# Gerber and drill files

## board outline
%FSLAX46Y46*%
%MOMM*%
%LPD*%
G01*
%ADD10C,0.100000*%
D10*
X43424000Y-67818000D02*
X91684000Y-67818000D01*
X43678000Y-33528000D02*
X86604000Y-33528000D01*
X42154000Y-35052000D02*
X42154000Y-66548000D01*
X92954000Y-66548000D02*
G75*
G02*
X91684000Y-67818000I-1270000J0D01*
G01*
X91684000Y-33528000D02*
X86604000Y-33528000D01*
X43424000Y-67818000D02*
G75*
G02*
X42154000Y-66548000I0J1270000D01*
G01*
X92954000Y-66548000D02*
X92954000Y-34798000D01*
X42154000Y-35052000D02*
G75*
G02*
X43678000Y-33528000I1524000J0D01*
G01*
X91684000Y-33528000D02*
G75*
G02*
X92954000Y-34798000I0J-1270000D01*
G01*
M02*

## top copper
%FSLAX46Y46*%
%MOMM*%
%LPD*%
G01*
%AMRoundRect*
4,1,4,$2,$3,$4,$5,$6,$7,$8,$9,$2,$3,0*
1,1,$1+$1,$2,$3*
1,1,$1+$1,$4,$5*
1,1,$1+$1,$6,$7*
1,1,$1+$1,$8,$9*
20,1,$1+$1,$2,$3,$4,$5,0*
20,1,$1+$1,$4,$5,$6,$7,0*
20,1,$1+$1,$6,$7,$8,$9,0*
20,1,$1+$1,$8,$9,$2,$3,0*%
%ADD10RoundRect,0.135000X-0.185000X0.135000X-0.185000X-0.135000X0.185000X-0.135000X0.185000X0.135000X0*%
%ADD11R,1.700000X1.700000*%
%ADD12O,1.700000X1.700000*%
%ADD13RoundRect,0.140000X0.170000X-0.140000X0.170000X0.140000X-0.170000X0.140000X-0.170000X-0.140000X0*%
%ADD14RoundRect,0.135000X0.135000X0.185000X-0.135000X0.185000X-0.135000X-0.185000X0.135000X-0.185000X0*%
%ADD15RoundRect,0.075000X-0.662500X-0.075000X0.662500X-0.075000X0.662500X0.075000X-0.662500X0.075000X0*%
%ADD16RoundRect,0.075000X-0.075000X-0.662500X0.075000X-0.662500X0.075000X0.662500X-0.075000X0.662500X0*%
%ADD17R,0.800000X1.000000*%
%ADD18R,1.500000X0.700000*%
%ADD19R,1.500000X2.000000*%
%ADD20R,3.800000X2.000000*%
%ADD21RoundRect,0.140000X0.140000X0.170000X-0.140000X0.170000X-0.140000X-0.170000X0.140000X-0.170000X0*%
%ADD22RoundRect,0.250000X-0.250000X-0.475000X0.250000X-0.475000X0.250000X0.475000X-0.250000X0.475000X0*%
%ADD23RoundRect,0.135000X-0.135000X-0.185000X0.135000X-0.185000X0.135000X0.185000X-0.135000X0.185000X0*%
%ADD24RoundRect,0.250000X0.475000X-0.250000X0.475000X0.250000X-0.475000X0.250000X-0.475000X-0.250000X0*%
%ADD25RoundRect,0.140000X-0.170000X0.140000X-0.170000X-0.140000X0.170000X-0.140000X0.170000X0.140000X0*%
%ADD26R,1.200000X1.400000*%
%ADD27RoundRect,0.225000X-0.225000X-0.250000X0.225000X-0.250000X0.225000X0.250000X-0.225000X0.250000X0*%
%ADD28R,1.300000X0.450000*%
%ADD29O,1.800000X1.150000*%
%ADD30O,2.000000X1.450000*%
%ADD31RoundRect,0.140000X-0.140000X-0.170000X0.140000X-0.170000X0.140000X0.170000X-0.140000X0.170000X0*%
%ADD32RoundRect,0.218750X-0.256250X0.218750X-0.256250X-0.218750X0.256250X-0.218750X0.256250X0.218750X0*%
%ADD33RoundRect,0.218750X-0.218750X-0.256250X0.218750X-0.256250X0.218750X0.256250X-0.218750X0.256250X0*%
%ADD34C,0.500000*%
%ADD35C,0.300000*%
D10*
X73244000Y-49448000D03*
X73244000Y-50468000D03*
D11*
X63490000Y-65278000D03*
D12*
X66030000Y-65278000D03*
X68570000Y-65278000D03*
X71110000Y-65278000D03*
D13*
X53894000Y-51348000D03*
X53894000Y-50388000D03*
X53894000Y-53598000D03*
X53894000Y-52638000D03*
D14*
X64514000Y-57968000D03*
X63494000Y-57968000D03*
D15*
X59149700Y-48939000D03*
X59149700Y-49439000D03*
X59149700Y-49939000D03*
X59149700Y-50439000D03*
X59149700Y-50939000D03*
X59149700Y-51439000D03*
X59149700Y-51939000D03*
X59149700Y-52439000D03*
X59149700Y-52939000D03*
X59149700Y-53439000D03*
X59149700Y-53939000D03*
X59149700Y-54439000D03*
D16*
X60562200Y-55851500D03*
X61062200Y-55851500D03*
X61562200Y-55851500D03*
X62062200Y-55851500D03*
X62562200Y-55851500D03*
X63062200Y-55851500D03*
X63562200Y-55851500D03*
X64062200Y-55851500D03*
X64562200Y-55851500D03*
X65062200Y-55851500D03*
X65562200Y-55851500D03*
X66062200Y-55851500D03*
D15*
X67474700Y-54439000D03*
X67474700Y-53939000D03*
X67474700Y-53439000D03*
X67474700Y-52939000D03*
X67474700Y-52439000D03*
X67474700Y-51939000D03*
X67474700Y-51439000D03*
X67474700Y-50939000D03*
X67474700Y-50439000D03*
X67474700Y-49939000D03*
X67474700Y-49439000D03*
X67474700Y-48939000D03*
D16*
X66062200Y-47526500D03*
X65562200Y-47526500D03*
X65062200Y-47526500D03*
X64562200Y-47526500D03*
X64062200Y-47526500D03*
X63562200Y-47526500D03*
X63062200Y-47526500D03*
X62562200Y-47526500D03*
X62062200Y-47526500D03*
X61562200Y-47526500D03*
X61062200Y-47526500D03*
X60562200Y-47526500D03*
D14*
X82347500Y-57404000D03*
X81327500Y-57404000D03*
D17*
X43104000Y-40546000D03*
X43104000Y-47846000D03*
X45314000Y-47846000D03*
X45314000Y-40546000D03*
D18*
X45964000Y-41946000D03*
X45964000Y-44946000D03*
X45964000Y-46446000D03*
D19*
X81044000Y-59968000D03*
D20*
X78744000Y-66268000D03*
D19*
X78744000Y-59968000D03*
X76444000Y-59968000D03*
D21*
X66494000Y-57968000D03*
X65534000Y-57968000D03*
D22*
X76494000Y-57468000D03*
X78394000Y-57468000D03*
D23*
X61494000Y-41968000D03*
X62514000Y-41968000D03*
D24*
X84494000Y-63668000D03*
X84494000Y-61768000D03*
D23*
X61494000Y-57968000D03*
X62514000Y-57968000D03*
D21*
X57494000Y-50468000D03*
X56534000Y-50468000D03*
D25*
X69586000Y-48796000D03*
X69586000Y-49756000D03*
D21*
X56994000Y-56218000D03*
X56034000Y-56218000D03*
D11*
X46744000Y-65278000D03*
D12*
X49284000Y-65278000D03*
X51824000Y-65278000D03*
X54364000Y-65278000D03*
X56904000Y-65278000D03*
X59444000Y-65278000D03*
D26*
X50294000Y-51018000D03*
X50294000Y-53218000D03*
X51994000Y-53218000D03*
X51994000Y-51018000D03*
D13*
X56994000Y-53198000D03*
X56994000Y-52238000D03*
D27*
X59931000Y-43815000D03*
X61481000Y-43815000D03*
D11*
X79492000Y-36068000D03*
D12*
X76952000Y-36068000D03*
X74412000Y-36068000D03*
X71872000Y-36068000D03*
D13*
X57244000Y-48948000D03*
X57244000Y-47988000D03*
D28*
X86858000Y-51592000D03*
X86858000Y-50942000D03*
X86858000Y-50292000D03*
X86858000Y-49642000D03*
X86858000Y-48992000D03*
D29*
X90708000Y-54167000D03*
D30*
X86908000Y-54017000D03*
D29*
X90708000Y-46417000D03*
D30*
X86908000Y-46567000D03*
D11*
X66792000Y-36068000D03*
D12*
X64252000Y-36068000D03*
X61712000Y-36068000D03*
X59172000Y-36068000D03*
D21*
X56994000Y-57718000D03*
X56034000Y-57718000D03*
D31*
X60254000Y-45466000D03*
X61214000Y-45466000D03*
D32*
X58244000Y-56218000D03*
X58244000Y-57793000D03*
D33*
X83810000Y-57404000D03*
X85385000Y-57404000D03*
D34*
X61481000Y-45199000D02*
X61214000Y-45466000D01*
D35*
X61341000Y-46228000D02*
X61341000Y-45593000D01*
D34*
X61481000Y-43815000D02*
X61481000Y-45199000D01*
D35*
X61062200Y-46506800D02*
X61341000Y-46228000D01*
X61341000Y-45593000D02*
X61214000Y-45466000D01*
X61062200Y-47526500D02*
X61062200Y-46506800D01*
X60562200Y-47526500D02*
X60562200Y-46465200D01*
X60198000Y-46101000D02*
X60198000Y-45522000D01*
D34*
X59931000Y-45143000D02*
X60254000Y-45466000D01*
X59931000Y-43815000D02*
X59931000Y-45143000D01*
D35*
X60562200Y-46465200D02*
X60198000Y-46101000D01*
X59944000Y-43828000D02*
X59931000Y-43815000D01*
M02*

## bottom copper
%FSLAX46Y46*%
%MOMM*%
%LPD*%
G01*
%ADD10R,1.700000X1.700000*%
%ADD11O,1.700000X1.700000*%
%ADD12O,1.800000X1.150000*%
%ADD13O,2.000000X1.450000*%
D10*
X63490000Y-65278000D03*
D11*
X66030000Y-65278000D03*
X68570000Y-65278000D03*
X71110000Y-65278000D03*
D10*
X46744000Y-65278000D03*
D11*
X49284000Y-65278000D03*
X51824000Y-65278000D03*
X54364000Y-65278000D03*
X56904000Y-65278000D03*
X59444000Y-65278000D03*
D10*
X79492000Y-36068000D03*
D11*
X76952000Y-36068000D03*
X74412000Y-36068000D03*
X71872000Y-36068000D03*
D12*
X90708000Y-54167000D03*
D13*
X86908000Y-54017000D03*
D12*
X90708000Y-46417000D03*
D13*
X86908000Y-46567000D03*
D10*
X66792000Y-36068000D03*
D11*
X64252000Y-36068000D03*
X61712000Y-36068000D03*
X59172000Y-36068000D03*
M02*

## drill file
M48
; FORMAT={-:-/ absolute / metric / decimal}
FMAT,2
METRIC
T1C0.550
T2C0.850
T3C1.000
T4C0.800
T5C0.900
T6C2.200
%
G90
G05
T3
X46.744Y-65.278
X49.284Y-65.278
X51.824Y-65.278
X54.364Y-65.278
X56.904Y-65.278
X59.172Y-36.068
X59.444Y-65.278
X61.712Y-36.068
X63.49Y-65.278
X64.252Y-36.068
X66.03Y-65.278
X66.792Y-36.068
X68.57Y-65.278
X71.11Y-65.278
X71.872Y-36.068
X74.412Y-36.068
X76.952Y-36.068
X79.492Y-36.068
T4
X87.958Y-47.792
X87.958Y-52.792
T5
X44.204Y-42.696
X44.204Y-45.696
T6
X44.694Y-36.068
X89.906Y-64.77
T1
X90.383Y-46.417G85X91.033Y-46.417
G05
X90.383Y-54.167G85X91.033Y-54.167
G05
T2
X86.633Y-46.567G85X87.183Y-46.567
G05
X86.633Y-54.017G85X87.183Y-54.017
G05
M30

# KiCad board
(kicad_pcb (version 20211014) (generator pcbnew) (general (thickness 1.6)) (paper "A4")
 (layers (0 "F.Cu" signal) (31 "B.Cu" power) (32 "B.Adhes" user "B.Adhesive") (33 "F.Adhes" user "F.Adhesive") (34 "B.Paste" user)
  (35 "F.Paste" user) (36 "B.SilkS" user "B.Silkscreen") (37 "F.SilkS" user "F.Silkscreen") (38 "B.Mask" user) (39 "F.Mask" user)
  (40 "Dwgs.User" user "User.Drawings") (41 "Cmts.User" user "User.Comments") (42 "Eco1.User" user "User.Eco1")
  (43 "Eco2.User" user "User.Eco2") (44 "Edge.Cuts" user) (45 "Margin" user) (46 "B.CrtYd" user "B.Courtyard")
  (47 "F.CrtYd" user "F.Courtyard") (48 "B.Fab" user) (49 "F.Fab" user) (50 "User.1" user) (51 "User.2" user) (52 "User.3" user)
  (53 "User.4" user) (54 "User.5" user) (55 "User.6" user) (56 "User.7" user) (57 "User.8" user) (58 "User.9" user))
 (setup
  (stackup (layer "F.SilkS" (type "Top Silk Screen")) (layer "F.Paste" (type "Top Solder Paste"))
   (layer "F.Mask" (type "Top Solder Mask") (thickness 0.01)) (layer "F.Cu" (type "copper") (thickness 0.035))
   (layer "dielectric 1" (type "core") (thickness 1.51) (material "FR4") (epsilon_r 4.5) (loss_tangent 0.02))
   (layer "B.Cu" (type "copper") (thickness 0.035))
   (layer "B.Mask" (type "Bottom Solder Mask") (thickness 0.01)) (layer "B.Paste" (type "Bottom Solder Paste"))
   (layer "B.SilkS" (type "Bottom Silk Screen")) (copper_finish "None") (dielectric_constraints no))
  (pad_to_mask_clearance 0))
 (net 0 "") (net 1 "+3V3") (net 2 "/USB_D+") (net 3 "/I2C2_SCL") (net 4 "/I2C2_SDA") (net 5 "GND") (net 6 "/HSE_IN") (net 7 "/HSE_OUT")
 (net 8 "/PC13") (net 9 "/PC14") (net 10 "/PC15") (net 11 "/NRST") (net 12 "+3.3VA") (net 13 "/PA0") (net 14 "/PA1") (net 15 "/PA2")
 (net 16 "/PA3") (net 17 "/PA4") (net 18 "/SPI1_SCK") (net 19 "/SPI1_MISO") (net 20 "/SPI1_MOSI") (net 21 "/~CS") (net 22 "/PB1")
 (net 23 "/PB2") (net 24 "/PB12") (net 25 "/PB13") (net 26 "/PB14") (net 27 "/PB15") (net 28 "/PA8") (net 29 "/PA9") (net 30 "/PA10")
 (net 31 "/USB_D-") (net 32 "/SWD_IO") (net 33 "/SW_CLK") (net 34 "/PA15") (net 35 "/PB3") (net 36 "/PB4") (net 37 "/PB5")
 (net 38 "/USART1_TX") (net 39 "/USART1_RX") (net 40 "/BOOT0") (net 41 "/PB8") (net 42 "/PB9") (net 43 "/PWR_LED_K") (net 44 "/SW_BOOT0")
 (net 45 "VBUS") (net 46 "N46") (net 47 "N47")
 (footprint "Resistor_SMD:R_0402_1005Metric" (layer "F.Cu") (at 73.244 49.958 -90)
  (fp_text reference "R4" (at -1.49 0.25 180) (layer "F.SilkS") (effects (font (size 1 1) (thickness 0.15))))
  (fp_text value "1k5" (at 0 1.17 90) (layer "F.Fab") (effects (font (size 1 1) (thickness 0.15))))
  (pad "1" smd roundrect locked (at -0.51 0 270) (size 0.54 0.64) (layers "F.Cu" "F.Paste" "F.Mask") (roundrect_rratio 0.25) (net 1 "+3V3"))
  (pad "2" smd roundrect locked (at 0.51 0 270) (size 0.54 0.64) (layers "F.Cu" "F.Paste" "F.Mask") (roundrect_rratio 0.25)
   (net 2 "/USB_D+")))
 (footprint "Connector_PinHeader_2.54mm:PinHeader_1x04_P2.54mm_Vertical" (layer "F.Cu") (at 63.49 65.278 90)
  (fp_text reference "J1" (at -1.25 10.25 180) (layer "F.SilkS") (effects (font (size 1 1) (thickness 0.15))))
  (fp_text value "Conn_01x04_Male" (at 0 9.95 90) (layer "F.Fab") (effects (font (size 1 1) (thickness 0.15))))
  (pad "1" thru_hole rect locked (at 0 0 90) (size 1.7 1.7) (drill 1) (layers *.Cu *.Mask) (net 1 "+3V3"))
  (pad "2" thru_hole oval locked (at 0 2.54 90) (size 1.7 1.7) (drill 1) (layers *.Cu *.Mask) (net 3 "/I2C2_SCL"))
  (pad "3" thru_hole oval locked (at 0 5.08 90) (size 1.7 1.7) (drill 1) (layers *.Cu *.Mask) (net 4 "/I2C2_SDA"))
  (pad "4" thru_hole oval locked (at 0 7.62 90) (size 1.7 1.7) (drill 1) (layers *.Cu *.Mask) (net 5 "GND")))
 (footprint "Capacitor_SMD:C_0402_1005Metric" (layer "F.Cu") (at 53.894 50.868 90)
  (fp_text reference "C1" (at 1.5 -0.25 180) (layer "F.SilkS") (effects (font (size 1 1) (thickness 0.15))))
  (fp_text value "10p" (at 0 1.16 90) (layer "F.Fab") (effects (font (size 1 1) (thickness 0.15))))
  (pad "1" smd roundrect locked (at -0.48 0 90) (size 0.56 0.62) (layers "F.Cu" "F.Paste" "F.Mask") (roundrect_rratio 0.25)
   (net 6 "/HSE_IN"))
  (pad "2" smd roundrect locked (at 0.48 0 90) (size 0.56 0.62) (layers "F.Cu" "F.Paste" "F.Mask") (roundrect_rratio 0.25) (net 5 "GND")))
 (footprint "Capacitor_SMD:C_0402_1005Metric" (layer "F.Cu") (at 53.894 53.118 90)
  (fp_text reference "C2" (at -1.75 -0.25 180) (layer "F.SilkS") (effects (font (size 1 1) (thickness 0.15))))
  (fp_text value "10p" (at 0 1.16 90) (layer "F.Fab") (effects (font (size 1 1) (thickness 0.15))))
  (pad "1" smd roundrect locked (at -0.48 0 90) (size 0.56 0.62) (layers "F.Cu" "F.Paste" "F.Mask") (roundrect_rratio 0.25)
   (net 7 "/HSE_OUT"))
  (pad "2" smd roundrect locked (at 0.48 0 90) (size 0.56 0.62) (layers "F.Cu" "F.Paste" "F.Mask") (roundrect_rratio 0.25) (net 5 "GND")))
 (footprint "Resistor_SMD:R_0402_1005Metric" (layer "F.Cu") (at 64.004 57.968 180)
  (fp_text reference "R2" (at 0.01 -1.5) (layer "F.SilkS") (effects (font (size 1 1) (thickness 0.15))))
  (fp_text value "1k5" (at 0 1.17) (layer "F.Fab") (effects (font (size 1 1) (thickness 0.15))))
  (pad "1" smd roundrect locked (at -0.51 0 180) (size 0.54 0.64) (layers "F.Cu" "F.Paste" "F.Mask") (roundrect_rratio 0.25) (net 1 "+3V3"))
  (pad "2" smd roundrect locked (at 0.51 0 180) (size 0.54 0.64) (layers "F.Cu" "F.Paste" "F.Mask") (roundrect_rratio 0.25)
   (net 4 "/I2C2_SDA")))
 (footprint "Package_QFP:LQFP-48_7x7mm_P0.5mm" (layer "F.Cu") (at 63.3122 51.689)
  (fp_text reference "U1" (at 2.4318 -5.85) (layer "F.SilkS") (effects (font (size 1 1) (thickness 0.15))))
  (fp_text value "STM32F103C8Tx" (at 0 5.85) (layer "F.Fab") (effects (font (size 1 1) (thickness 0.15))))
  (pad "1" smd roundrect locked (at -4.1625 -2.75) (size 1.475 0.3) (layers "F.Cu" "F.Paste" "F.Mask") (roundrect_rratio 0.25)
   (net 1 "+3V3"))
  (pad "2" smd roundrect locked (at -4.1625 -2.25) (size 1.475 0.3) (layers "F.Cu" "F.Paste" "F.Mask") (roundrect_rratio 0.25)
   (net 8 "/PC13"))
  (pad "3" smd roundrect locked (at -4.1625 -1.75) (size 1.475 0.3) (layers "F.Cu" "F.Paste" "F.Mask") (roundrect_rratio 0.25)
   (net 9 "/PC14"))
  (pad "4" smd roundrect locked (at -4.1625 -1.25) (size 1.475 0.3) (layers "F.Cu" "F.Paste" "F.Mask") (roundrect_rratio 0.25)
   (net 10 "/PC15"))
  (pad "5" smd roundrect locked (at -4.1625 -0.75) (size 1.475 0.3) (layers "F.Cu" "F.Paste" "F.Mask") (roundrect_rratio 0.25)
   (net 6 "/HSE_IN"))
  (pad "6" smd roundrect locked (at -4.1625 -0.25) (size 1.475 0.3) (layers "F.Cu" "F.Paste" "F.Mask") (roundrect_rratio 0.25)
   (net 7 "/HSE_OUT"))
  (pad "7" smd roundrect locked (at -4.1625 0.25) (size 1.475 0.3) (layers "F.Cu" "F.Paste" "F.Mask") (roundrect_rratio 0.25)
   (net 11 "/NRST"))
  (pad "8" smd roundrect locked (at -4.1625 0.75) (size 1.475 0.3) (layers "F.Cu" "F.Paste" "F.Mask") (roundrect_rratio 0.25) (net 5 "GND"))
  (pad "9" smd roundrect locked (at -4.1625 1.25) (size 1.475 0.3) (layers "F.Cu" "F.Paste" "F.Mask") (roundrect_rratio 0.25)
   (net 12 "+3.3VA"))
  (pad "10" smd roundrect locked (at -4.1625 1.75) (size 1.475 0.3) (layers "F.Cu" "F.Paste" "F.Mask") (roundrect_rratio 0.25)
   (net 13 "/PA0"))
  (pad "11" smd roundrect locked (at -4.1625 2.25) (size 1.475 0.3) (layers "F.Cu" "F.Paste" "F.Mask") (roundrect_rratio 0.25)
   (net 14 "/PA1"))
  (pad "12" smd roundrect locked (at -4.1625 2.75) (size 1.475 0.3) (layers "F.Cu" "F.Paste" "F.Mask") (roundrect_rratio 0.25)
   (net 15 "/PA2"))
  (pad "13" smd roundrect locked (at -2.75 4.1625) (size 0.3 1.475) (layers "F.Cu" "F.Paste" "F.Mask") (roundrect_rratio 0.25)
   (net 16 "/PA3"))
  (pad "14" smd roundrect locked (at -2.25 4.1625) (size 0.3 1.475) (layers "F.Cu" "F.Paste" "F.Mask") (roundrect_rratio 0.25)
   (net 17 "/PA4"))
  (pad "15" smd roundrect locked (at -1.75 4.1625) (size 0.3 1.475) (layers "F.Cu" "F.Paste" "F.Mask") (roundrect_rratio 0.25)
   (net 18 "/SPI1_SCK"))
  (pad "16" smd roundrect locked (at -1.25 4.1625) (size 0.3 1.475) (layers "F.Cu" "F.Paste" "F.Mask") (roundrect_rratio 0.25)
   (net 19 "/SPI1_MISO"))
  (pad "17" smd roundrect locked (at -0.75 4.1625) (size 0.3 1.475) (layers "F.Cu" "F.Paste" "F.Mask") (roundrect_rratio 0.25)
   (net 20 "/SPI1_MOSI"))
  (pad "18" smd roundrect locked (at -0.25 4.1625) (size 0.3 1.475) (layers "F.Cu" "F.Paste" "F.Mask") (roundrect_rratio 0.25)
   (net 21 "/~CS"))
  (pad "19" smd roundrect locked (at 0.25 4.1625) (size 0.3 1.475) (layers "F.Cu" "F.Paste" "F.Mask") (roundrect_rratio 0.25)
   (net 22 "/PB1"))
  (pad "20" smd roundrect locked (at 0.75 4.1625) (size 0.3 1.475) (layers "F.Cu" "F.Paste" "F.Mask") (roundrect_rratio 0.25)
   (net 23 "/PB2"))
  (pad "21" smd roundrect locked (at 1.25 4.1625) (size 0.3 1.475) (layers "F.Cu" "F.Paste" "F.Mask") (roundrect_rratio 0.25)
   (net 3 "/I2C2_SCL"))
  (pad "22" smd roundrect locked (at 1.75 4.1625) (size 0.3 1.475) (layers "F.Cu" "F.Paste" "F.Mask") (roundrect_rratio 0.25)
   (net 4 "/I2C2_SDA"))
  (pad "23" smd roundrect locked (at 2.25 4.1625) (size 0.3 1.475) (layers "F.Cu" "F.Paste" "F.Mask") (roundrect_rratio 0.25) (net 5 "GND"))
  (pad "24" smd roundrect locked (at 2.75 4.1625) (size 0.3 1.475) (layers "F.Cu" "F.Paste" "F.Mask") (roundrect_rratio 0.25) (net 1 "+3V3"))
  (pad "25" smd roundrect locked (at 4.1625 2.75) (size 1.475 0.3) (layers "F.Cu" "F.Paste" "F.Mask") (roundrect_rratio 0.25)
   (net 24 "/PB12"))
  (pad "26" smd roundrect locked (at 4.1625 2.25) (size 1.475 0.3) (layers "F.Cu" "F.Paste" "F.Mask") (roundrect_rratio 0.25)
   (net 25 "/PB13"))
  (pad "27" smd roundrect locked (at 4.1625 1.75) (size 1.475 0.3) (layers "F.Cu" "F.Paste" "F.Mask") (roundrect_rratio 0.25)
   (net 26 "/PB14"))
  (pad "28" smd roundrect locked (at 4.1625 1.25) (size 1.475 0.3) (layers "F.Cu" "F.Paste" "F.Mask") (roundrect_rratio 0.25)
   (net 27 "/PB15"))
  (pad "29" smd roundrect locked (at 4.1625 0.75) (size 1.475 0.3) (layers "F.Cu" "F.Paste" "F.Mask") (roundrect_rratio 0.25)
   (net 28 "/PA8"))
  (pad "30" smd roundrect locked (at 4.1625 0.25) (size 1.475 0.3) (layers "F.Cu" "F.Paste" "F.Mask") (roundrect_rratio 0.25)
   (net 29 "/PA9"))
  (pad "31" smd roundrect locked (at 4.1625 -0.25) (size 1.475 0.3) (layers "F.Cu" "F.Paste" "F.Mask") (roundrect_rratio 0.25)
   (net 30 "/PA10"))
  (pad "32" smd roundrect locked (at 4.1625 -0.75) (size 1.475 0.3) (layers "F.Cu" "F.Paste" "F.Mask") (roundrect_rratio 0.25)
   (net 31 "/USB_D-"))
  (pad "33" smd roundrect locked (at 4.1625 -1.25) (size 1.475 0.3) (layers "F.Cu" "F.Paste" "F.Mask") (roundrect_rratio 0.25)
   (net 2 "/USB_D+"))
  (pad "34" smd roundrect locked (at 4.1625 -1.75) (size 1.475 0.3) (layers "F.Cu" "F.Paste" "F.Mask") (roundrect_rratio 0.25)
   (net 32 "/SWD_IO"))
  (pad "35" smd roundrect locked (at 4.1625 -2.25) (size 1.475 0.3) (layers "F.Cu" "F.Paste" "F.Mask") (roundrect_rratio 0.25) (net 5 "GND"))
  (pad "36" smd roundrect locked (at 4.1625 -2.75) (size 1.475 0.3) (layers "F.Cu" "F.Paste" "F.Mask") (roundrect_rratio 0.25)
   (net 1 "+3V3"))
  (pad "37" smd roundrect locked (at 2.75 -4.1625) (size 0.3 1.475) (layers "F.Cu" "F.Paste" "F.Mask") (roundrect_rratio 0.25)
   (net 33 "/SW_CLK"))
  (pad "38" smd roundrect locked (at 2.25 -4.1625) (size 0.3 1.475) (layers "F.Cu" "F.Paste" "F.Mask") (roundrect_rratio 0.25)
   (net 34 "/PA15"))
  (pad "39" smd roundrect locked (at 1.75 -4.1625) (size 0.3 1.475) (layers "F.Cu" "F.Paste" "F.Mask") (roundrect_rratio 0.25)
   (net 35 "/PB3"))
  (pad "40" smd roundrect locked (at 1.25 -4.1625) (size 0.3 1.475) (layers "F.Cu" "F.Paste" "F.Mask") (roundrect_rratio 0.25)
   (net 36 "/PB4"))
  (pad "41" smd roundrect locked (at 0.75 -4.1625) (size 0.3 1.475) (layers "F.Cu" "F.Paste" "F.Mask") (roundrect_rratio 0.25)
   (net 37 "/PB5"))
  (pad "42" smd roundrect locked (at 0.25 -4.1625) (size 0.3 1.475) (layers "F.Cu" "F.Paste" "F.Mask") (roundrect_rratio 0.25)
   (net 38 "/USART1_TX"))
  (pad "43" smd roundrect locked (at -0.25 -4.1625) (size 0.3 1.475) (layers "F.Cu" "F.Paste" "F.Mask") (roundrect_rratio 0.25)
   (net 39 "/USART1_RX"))
  (pad "44" smd roundrect locked (at -0.75 -4.1625) (size 0.3 1.475) (layers "F.Cu" "F.Paste" "F.Mask") (roundrect_rratio 0.25)
   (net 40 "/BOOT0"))
  (pad "45" smd roundrect locked (at -1.25 -4.1625) (size 0.3 1.475) (layers "F.Cu" "F.Paste" "F.Mask") (roundrect_rratio 0.25)
   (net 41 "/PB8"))
  (pad "46" smd roundrect locked (at -1.75 -4.1625) (size 0.3 1.475) (layers "F.Cu" "F.Paste" "F.Mask") (roundrect_rratio 0.25)
   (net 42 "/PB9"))
  (pad "47" smd roundrect locked (at -2.25 -4.1625) (size 0.3 1.475) (layers "F.Cu" "F.Paste" "F.Mask") (roundrect_rratio 0.25)
   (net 5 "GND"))
  (pad "48" smd roundrect locked (at -2.75 -4.1625) (size 0.3 1.475) (layers "F.Cu" "F.Paste" "F.Mask") (roundrect_rratio 0.25)
   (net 1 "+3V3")))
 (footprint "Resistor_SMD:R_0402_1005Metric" (layer "F.Cu") (at 81.8375 57.404 180)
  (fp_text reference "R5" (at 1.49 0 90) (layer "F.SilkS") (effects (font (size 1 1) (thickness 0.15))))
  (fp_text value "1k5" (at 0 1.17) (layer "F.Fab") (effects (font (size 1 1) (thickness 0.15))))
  (pad "1" smd roundrect locked (at -0.51 0 180) (size 0.54 0.64) (layers "F.Cu" "F.Paste" "F.Mask") (roundrect_rratio 0.25)
   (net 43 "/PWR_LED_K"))
  (pad "2" smd roundrect locked (at 0.51 0 180) (size 0.54 0.64) (layers "F.Cu" "F.Paste" "F.Mask") (roundrect_rratio 0.25) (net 5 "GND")))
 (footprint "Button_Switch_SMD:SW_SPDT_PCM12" (layer "F.Cu") (at 44.534 44.196 -90)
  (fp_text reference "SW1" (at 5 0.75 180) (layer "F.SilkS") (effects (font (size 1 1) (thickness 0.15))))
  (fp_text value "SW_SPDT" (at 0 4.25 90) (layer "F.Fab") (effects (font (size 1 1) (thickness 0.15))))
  (pad "" smd rect (at -3.65 1.43 270) (size 1 0.8) (layers "F.Cu" "F.Paste" "F.Mask"))
  (pad "" smd rect (at 3.65 1.43 270) (size 1 0.8) (layers "F.Cu" "F.Paste" "F.Mask"))
  (pad "" np_thru_hole circle (at 1.5 0.33 270) (size 0.9 0.9) (drill 0.9) (layers *.Cu *.Mask))
  (pad "" smd rect (at 3.65 -0.78 270) (size 1 0.8) (layers "F.Cu" "F.Paste" "F.Mask"))
  (pad "" smd rect (at -3.65 -0.78 270) (size 1 0.8) (layers "F.Cu" "F.Paste" "F.Mask"))
  (pad "" np_thru_hole circle (at -1.5 0.33 270) (size 0.9 0.9) (drill 0.9) (layers *.Cu *.Mask))
  (pad "1" smd rect (at -2.25 -1.43 270) (size 0.7 1.5) (layers "F.Cu" "F.Paste" "F.Mask") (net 5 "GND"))
  (pad "2" smd rect (at 0.75 -1.43 270) (size 0.7 1.5) (layers "F.Cu" "F.Paste" "F.Mask") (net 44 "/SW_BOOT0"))
  (pad "3" smd rect (at 2.25 -1.43 270) (size 0.7 1.5) (layers "F.Cu" "F.Paste" "F.Mask") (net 1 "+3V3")))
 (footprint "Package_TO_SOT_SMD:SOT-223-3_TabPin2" (layer "F.Cu") (at 78.744 63.118 -90)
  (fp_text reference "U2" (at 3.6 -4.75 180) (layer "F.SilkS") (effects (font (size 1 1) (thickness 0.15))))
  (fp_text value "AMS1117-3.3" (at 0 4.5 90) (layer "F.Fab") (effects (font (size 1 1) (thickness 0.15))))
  (pad "1" smd rect locked (at -3.15 -2.3 270) (size 2 1.5) (layers "F.Cu" "F.Paste" "F.Mask") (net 5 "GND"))
  (pad "2" smd rect locked (at 3.15 0 270) (size 2 3.8) (layers "F.Cu" "F.Paste" "F.Mask") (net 1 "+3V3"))
  (pad "2" smd rect locked (at -3.15 0 270) (size 2 1.5) (layers "F.Cu" "F.Paste" "F.Mask") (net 1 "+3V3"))
  (pad "3" smd rect locked (at -3.15 2.3 270) (size 2 1.5) (layers "F.Cu" "F.Paste" "F.Mask") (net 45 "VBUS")))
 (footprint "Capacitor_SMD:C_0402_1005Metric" (layer "F.Cu") (at 66.014 57.968 180)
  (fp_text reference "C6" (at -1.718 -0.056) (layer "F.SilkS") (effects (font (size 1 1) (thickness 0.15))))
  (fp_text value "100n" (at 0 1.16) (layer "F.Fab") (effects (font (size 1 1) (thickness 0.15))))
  (pad "1" smd roundrect locked (at -0.48 0 180) (size 0.56 0.62) (layers "F.Cu" "F.Paste" "F.Mask") (roundrect_rratio 0.25) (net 1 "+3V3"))
  (pad "2" smd roundrect locked (at 0.48 0 180) (size 0.56 0.62) (layers "F.Cu" "F.Paste" "F.Mask") (roundrect_rratio 0.25) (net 5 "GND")))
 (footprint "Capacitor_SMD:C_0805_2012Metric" (layer "F.Cu") (at 77.444 57.468)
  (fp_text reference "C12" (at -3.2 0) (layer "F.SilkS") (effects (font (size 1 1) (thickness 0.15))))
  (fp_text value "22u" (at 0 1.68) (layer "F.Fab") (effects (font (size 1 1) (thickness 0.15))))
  (pad "1" smd roundrect locked (at -0.95 0) (size 1 1.45) (layers "F.Cu" "F.Paste" "F.Mask") (roundrect_rratio 0.25) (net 45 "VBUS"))
  (pad "2" smd roundrect locked (at 0.95 0) (size 1 1.45) (layers "F.Cu" "F.Paste" "F.Mask") (roundrect_rratio 0.25) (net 5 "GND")))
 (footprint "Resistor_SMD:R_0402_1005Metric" (layer "F.Cu") (at 62.004 41.968)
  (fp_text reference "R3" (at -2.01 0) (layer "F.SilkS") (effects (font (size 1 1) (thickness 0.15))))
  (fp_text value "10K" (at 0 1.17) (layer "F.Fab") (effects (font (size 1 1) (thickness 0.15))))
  (pad "1" smd roundrect locked (at -0.51 0) (size 0.54 0.64) (layers "F.Cu" "F.Paste" "F.Mask") (roundrect_rratio 0.25)
   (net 44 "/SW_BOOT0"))
  (pad "2" smd roundrect locked (at 0.51 0) (size 0.54 0.64) (layers "F.Cu" "F.Paste" "F.Mask") (roundrect_rratio 0.25) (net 40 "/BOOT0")))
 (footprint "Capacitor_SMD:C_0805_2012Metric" (layer "F.Cu") (at 84.494 62.718 90)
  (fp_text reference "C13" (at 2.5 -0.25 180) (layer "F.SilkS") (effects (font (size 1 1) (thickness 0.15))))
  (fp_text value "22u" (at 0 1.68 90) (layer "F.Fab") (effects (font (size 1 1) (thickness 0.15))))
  (pad "1" smd roundrect locked (at -0.95 0 90) (size 1 1.45) (layers "F.Cu" "F.Paste" "F.Mask") (roundrect_rratio 0.25) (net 1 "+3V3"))
  (pad "2" smd roundrect locked (at 0.95 0 90) (size 1 1.45) (layers "F.Cu" "F.Paste" "F.Mask") (roundrect_rratio 0.25) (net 5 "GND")))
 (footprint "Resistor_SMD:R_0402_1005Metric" (layer "F.Cu") (at 62.004 57.968)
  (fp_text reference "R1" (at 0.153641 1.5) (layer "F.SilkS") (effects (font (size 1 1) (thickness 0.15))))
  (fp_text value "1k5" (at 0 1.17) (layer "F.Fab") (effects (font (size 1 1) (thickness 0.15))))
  (pad "1" smd roundrect locked (at -0.51 0) (size 0.54 0.64) (layers "F.Cu" "F.Paste" "F.Mask") (roundrect_rratio 0.25) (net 1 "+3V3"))
  (pad "2" smd roundrect locked (at 0.51 0) (size 0.54 0.64) (layers "F.Cu" "F.Paste" "F.Mask") (roundrect_rratio 0.25) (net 3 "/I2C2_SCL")))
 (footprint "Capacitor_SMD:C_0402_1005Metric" (layer "F.Cu") (at 57.014 50.468 180)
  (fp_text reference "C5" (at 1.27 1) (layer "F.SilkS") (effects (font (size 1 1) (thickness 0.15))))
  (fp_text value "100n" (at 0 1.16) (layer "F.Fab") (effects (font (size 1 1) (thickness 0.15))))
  (pad "1" smd roundrect locked (at -0.48 0 180) (size 0.56 0.62) (layers "F.Cu" "F.Paste" "F.Mask") (roundrect_rratio 0.25)
   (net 11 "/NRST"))
  (pad "2" smd roundrect locked (at 0.48 0 180) (size 0.56 0.62) (layers "F.Cu" "F.Paste" "F.Mask") (roundrect_rratio 0.25) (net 5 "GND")))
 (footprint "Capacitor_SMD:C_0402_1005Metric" (layer "F.Cu") (at 69.586 49.276 -90)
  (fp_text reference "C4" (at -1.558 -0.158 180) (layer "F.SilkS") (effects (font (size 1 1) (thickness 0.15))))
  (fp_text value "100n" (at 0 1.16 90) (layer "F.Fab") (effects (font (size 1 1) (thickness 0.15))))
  (pad "1" smd roundrect locked (at -0.48 0 270) (size 0.56 0.62) (layers "F.Cu" "F.Paste" "F.Mask") (roundrect_rratio 0.25) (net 1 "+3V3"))
  (pad "2" smd roundrect locked (at 0.48 0 270) (size 0.56 0.62) (layers "F.Cu" "F.Paste" "F.Mask") (roundrect_rratio 0.25) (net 5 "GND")))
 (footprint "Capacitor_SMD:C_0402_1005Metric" (layer "F.Cu") (at 56.514 56.218 180)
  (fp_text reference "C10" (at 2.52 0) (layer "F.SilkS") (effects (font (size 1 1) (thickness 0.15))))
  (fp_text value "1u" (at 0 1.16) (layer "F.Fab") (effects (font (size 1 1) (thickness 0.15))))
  (pad "1" smd roundrect locked (at -0.48 0 180) (size 0.56 0.62) (layers "F.Cu" "F.Paste" "F.Mask") (roundrect_rratio 0.25)
   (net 12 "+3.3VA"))
  (pad "2" smd roundrect locked (at 0.48 0 180) (size 0.56 0.62) (layers "F.Cu" "F.Paste" "F.Mask") (roundrect_rratio 0.25) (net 5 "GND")))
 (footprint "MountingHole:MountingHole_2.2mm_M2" (layer "F.Cu") (at 89.906 64.77)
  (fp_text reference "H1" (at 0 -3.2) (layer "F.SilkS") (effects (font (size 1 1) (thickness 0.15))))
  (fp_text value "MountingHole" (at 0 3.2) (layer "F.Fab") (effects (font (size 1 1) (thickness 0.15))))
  (pad "" np_thru_hole circle locked (at 0 0) (size 2.2 2.2) (drill 2.2) (layers *.Cu *.Mask)))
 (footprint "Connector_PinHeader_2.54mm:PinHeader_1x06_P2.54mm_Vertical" (layer "F.Cu") (at 46.744 65.278 90)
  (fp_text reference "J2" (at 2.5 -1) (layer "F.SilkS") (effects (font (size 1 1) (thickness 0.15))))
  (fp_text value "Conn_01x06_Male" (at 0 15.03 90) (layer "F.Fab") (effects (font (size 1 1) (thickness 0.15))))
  (pad "1" thru_hole rect locked (at 0 0 90) (size 1.7 1.7) (drill 1) (layers *.Cu *.Mask) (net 1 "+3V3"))
  (pad "2" thru_hole oval locked (at 0 2.54 90) (size 1.7 1.7) (drill 1) (layers *.Cu *.Mask) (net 18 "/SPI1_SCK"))
  (pad "3" thru_hole oval locked (at 0 5.08 90) (size 1.7 1.7) (drill 1) (layers *.Cu *.Mask) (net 19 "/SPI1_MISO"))
  (pad "4" thru_hole oval locked (at 0 7.62 90) (size 1.7 1.7) (drill 1) (layers *.Cu *.Mask) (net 20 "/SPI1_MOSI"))
  (pad "5" thru_hole oval locked (at 0 10.16 90) (size 1.7 1.7) (drill 1) (layers *.Cu *.Mask) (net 21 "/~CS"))
  (pad "6" thru_hole oval locked (at 0 12.7 90) (size 1.7 1.7) (drill 1) (layers *.Cu *.Mask) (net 5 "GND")))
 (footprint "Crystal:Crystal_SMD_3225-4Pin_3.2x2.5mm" (layer "F.Cu") (at 51.144 52.118 -90)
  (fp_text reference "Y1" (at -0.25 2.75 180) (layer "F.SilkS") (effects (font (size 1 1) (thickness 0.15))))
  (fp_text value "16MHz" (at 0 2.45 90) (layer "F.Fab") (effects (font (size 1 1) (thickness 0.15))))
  (pad "1" smd rect locked (at -1.1 0.85 270) (size 1.4 1.2) (layers "F.Cu" "F.Paste" "F.Mask") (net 6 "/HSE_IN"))
  (pad "2" smd rect locked (at 1.1 0.85 270) (size 1.4 1.2) (layers "F.Cu" "F.Paste" "F.Mask") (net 5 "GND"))
  (pad "3" smd rect locked (at 1.1 -0.85 270) (size 1.4 1.2) (layers "F.Cu" "F.Paste" "F.Mask") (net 7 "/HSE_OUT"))
  (pad "4" smd rect locked (at -1.1 -0.85 270) (size 1.4 1.2) (layers "F.Cu" "F.Paste" "F.Mask") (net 5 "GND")))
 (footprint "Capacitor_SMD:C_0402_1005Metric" (layer "F.Cu") (at 56.994 52.718 90)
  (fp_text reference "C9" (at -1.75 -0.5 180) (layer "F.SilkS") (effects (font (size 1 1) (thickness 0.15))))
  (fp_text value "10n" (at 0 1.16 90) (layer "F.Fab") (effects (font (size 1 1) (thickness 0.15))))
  (pad "1" smd roundrect locked (at -0.48 0 90) (size 0.56 0.62) (layers "F.Cu" "F.Paste" "F.Mask") (roundrect_rratio 0.25)
   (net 12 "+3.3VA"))
  (pad "2" smd roundrect locked (at 0.48 0 90) (size 0.56 0.62) (layers "F.Cu" "F.Paste" "F.Mask") (roundrect_rratio 0.25) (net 5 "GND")))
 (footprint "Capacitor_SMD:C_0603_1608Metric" (layer "F.Cu") (at 60.706 43.815)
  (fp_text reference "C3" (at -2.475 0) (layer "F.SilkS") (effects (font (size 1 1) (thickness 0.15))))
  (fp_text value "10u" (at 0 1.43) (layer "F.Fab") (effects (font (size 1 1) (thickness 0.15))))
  (pad "1" smd roundrect locked (at -0.775 0) (size 0.9 0.95) (layers "F.Cu" "F.Paste" "F.Mask") (roundrect_rratio 0.25) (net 1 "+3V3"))
  (pad "2" smd roundrect locked (at 0.775 0) (size 0.9 0.95) (layers "F.Cu" "F.Paste" "F.Mask") (roundrect_rratio 0.25) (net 5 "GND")))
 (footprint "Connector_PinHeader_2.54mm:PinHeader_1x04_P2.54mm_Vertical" (layer "F.Cu") (at 79.492 36.068 -90)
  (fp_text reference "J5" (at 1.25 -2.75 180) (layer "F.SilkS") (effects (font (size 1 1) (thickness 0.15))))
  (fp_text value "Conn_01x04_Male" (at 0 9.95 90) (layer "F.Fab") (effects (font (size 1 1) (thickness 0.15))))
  (pad "1" thru_hole rect locked (at 0 0 270) (size 1.7 1.7) (drill 1) (layers *.Cu *.Mask) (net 1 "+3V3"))
  (pad "2" thru_hole oval locked (at 0 2.54 270) (size 1.7 1.7) (drill 1) (layers *.Cu *.Mask) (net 32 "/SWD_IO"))
  (pad "3" thru_hole oval locked (at 0 5.08 270) (size 1.7 1.7) (drill 1) (layers *.Cu *.Mask) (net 33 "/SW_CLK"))
  (pad "4" thru_hole oval locked (at 0 7.62 270) (size 1.7 1.7) (drill 1) (layers *.Cu *.Mask) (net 5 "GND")))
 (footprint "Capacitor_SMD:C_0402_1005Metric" (layer "F.Cu") (at 57.244 48.468 90)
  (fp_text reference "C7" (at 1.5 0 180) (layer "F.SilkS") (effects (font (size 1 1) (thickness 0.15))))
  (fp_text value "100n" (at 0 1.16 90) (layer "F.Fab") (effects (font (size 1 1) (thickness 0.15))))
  (pad "1" smd roundrect locked (at -0.48 0 90) (size 0.56 0.62) (layers "F.Cu" "F.Paste" "F.Mask") (roundrect_rratio 0.25) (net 1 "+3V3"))
  (pad "2" smd roundrect locked (at 0.48 0 90) (size 0.56 0.62) (layers "F.Cu" "F.Paste" "F.Mask") (roundrect_rratio 0.25) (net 5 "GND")))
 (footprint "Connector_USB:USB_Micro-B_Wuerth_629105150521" (layer "F.Cu") (at 88.758 50.292 90)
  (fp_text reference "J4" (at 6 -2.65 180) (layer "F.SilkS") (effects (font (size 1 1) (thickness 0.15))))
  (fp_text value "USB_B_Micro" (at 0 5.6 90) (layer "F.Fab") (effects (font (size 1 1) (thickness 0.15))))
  (pad "" np_thru_hole oval locked (at 2.5 -0.8 90) (size 0.8 0.8) (drill 0.8) (layers *.Cu *.Mask))
  (pad "" np_thru_hole oval locked (at -2.5 -0.8 90) (size 0.8 0.8) (drill 0.8) (layers *.Cu *.Mask))
  (pad "1" smd rect locked (at -1.3 -1.9 90) (size 0.45 1.3) (layers "F.Cu" "F.Paste" "F.Mask") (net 45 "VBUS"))
  (pad "2" smd rect locked (at -0.65 -1.9 90) (size 0.45 1.3) (layers "F.Cu" "F.Paste" "F.Mask") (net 31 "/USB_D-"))
  (pad "3" smd rect locked (at 0 -1.9 90) (size 0.45 1.3) (layers "F.Cu" "F.Paste" "F.Mask") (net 2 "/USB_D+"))
  (pad "4" smd rect locked (at 0.65 -1.9 90) (size 0.45 1.3) (layers "F.Cu" "F.Paste" "F.Mask") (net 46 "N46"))
  (pad "5" smd rect locked (at 1.3 -1.9 90) (size 0.45 1.3) (layers "F.Cu" "F.Paste" "F.Mask") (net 5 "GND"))
  (pad "6" thru_hole oval locked (at -3.875 1.95 90) (size 1.15 1.8) (drill oval 0.55 1.2) (layers *.Cu *.Mask) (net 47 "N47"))
  (pad "6" thru_hole oval locked (at -3.725 -1.85 90) (size 1.45 2) (drill oval 0.85 1.4) (layers *.Cu *.Mask) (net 47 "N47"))
  (pad "6" thru_hole oval locked (at 3.875 1.95 90) (size 1.15 1.8) (drill oval 0.55 1.2) (layers *.Cu *.Mask) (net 47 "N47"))
  (pad "6" thru_hole oval locked (at 3.725 -1.85 90) (size 1.45 2) (drill oval 0.85 1.4) (layers *.Cu *.Mask) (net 47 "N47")))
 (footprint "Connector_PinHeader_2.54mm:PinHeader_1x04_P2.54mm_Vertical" (layer "F.Cu") (at 66.792 36.068 -90)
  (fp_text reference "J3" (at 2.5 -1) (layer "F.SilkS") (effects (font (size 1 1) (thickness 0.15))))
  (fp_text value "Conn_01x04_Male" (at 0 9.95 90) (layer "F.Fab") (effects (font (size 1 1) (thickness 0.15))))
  (pad "1" thru_hole rect locked (at 0 0 270) (size 1.7 1.7) (drill 1) (layers *.Cu *.Mask) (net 1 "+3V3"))
  (pad "2" thru_hole oval locked (at 0 2.54 270) (size 1.7 1.7) (drill 1) (layers *.Cu *.Mask) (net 38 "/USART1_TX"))
  (pad "3" thru_hole oval locked (at 0 5.08 270) (size 1.7 1.7) (drill 1) (layers *.Cu *.Mask) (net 39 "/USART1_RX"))
  (pad "4" thru_hole oval locked (at 0 7.62 270) (size 1.7 1.7) (drill 1) (layers *.Cu *.Mask) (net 5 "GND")))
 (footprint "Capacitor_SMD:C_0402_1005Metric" (layer "F.Cu") (at 56.514 57.718 180)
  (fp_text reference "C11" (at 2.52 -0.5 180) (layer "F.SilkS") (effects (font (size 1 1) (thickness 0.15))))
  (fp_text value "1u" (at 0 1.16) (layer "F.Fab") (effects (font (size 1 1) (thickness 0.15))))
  (pad "1" smd roundrect locked (at -0.48 0 180) (size 0.56 0.62) (layers "F.Cu" "F.Paste" "F.Mask") (roundrect_rratio 0.25) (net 1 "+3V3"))
  (pad "2" smd roundrect locked (at 0.48 0 180) (size 0.56 0.62) (layers "F.Cu" "F.Paste" "F.Mask") (roundrect_rratio 0.25) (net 5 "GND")))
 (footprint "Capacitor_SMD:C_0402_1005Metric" (layer "F.Cu") (at 60.734 45.466)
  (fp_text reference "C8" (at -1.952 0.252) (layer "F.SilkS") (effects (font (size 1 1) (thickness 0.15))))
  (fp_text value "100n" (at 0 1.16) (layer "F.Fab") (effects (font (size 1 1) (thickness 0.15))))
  (pad "1" smd roundrect locked (at -0.48 0) (size 0.56 0.62) (layers "F.Cu" "F.Paste" "F.Mask") (roundrect_rratio 0.25) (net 1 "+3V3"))
  (pad "2" smd roundrect locked (at 0.48 0) (size 0.56 0.62) (layers "F.Cu" "F.Paste" "F.Mask") (roundrect_rratio 0.25) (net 5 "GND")))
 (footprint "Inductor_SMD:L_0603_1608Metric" (layer "F.Cu") (at 58.244 57.0055 -90)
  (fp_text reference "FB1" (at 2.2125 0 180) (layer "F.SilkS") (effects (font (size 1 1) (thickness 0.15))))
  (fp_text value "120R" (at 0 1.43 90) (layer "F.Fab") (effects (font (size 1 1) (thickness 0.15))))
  (pad "1" smd roundrect locked (at -0.7875 0 270) (size 0.875 0.95) (layers "F.Cu" "F.Paste" "F.Mask") (roundrect_rratio 0.25)
   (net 12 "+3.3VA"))
  (pad "2" smd roundrect locked (at 0.7875 0 270) (size 0.875 0.95) (layers "F.Cu" "F.Paste" "F.Mask") (roundrect_rratio 0.25)
   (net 1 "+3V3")))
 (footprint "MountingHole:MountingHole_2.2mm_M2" (layer "F.Cu") (at 44.694 36.068)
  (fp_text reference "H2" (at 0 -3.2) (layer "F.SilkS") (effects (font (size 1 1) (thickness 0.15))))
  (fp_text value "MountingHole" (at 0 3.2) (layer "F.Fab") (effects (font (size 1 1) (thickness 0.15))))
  (pad "" np_thru_hole circle locked (at 0 0) (size 2.2 2.2) (drill 2.2) (layers *.Cu *.Mask)))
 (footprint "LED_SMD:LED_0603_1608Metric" (layer "F.Cu") (at 84.5975 57.404)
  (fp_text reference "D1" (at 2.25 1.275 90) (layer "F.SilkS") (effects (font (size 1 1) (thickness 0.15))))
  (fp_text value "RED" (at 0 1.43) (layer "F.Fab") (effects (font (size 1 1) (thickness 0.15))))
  (pad "1" smd roundrect locked (at -0.7875 0) (size 0.875 0.95) (layers "F.Cu" "F.Paste" "F.Mask") (roundrect_rratio 0.25)
   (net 43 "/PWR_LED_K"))
  (pad "2" smd roundrect locked (at 0.7875 0) (size 0.875 0.95) (layers "F.Cu" "F.Paste" "F.Mask") (roundrect_rratio 0.25) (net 1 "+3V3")))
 (gr_line (start 43.424 67.818) (end 91.684 67.818) (layer "Edge.Cuts") (width 0.1))
 (gr_line (start 43.678 33.528) (end 86.604 33.528) (layer "Edge.Cuts") (width 0.1))
 (gr_line (start 42.154 35.052) (end 42.154 66.548) (layer "Edge.Cuts") (width 0.1))
 (gr_arc (start 92.954 66.548) (mid 92.582026 67.446026) (end 91.684 67.818) (layer "Edge.Cuts") (width 0.1))
 (gr_line (start 91.684 33.528) (end 86.604 33.528) (layer "Edge.Cuts") (width 0.1))
 (gr_arc (start 43.424 67.818) (mid 42.525974 67.446026) (end 42.154 66.548) (layer "Edge.Cuts") (width 0.1))
 (gr_line (start 92.954 66.548) (end 92.954 34.798) (layer "Edge.Cuts") (width 0.1))
 (gr_arc (start 42.154 35.052) (mid 42.600369 33.974369) (end 43.678 33.528) (layer "Edge.Cuts") (width 0.1))
 (gr_arc (start 91.684 33.528) (mid 92.582026 33.899974) (end 92.954 34.798) (layer "Edge.Cuts") (width 0.1))
 (segment (start 61.481 45.199) (end 61.214 45.466) (width 0.5) (layer "F.Cu") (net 5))
 (segment (start 61.341 46.228) (end 61.341 45.593) (width 0.3) (layer "F.Cu") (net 5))
 (segment (start 61.481 43.815) (end 61.481 45.199) (width 0.5) (layer "F.Cu") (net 5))
 (segment (start 61.0622 46.5068) (end 61.341 46.228) (width 0.3) (layer "F.Cu") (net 5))
 (segment (start 61.341 45.593) (end 61.214 45.466) (width 0.3) (layer "F.Cu") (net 5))
 (segment (start 61.0622 47.5265) (end 61.0622 46.5068) (width 0.3) (layer "F.Cu") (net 5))
 (segment (start 60.5622 47.5265) (end 60.5622 46.4652) (width 0.3) (layer "F.Cu") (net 1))
 (segment (start 60.198 46.101) (end 60.198 45.522) (width 0.3) (layer "F.Cu") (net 1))
 (segment (start 59.931 45.143) (end 60.254 45.466) (width 0.5) (layer "F.Cu") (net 1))
 (segment (start 59.931 43.815) (end 59.931 45.143) (width 0.5) (layer "F.Cu") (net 1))
 (segment (start 60.5622 46.4652) (end 60.198 46.101) (width 0.3) (layer "F.Cu") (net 1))
 (segment (start 59.944 43.828) (end 59.931 43.815) (width 0.3) (layer "F.Cu") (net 1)))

